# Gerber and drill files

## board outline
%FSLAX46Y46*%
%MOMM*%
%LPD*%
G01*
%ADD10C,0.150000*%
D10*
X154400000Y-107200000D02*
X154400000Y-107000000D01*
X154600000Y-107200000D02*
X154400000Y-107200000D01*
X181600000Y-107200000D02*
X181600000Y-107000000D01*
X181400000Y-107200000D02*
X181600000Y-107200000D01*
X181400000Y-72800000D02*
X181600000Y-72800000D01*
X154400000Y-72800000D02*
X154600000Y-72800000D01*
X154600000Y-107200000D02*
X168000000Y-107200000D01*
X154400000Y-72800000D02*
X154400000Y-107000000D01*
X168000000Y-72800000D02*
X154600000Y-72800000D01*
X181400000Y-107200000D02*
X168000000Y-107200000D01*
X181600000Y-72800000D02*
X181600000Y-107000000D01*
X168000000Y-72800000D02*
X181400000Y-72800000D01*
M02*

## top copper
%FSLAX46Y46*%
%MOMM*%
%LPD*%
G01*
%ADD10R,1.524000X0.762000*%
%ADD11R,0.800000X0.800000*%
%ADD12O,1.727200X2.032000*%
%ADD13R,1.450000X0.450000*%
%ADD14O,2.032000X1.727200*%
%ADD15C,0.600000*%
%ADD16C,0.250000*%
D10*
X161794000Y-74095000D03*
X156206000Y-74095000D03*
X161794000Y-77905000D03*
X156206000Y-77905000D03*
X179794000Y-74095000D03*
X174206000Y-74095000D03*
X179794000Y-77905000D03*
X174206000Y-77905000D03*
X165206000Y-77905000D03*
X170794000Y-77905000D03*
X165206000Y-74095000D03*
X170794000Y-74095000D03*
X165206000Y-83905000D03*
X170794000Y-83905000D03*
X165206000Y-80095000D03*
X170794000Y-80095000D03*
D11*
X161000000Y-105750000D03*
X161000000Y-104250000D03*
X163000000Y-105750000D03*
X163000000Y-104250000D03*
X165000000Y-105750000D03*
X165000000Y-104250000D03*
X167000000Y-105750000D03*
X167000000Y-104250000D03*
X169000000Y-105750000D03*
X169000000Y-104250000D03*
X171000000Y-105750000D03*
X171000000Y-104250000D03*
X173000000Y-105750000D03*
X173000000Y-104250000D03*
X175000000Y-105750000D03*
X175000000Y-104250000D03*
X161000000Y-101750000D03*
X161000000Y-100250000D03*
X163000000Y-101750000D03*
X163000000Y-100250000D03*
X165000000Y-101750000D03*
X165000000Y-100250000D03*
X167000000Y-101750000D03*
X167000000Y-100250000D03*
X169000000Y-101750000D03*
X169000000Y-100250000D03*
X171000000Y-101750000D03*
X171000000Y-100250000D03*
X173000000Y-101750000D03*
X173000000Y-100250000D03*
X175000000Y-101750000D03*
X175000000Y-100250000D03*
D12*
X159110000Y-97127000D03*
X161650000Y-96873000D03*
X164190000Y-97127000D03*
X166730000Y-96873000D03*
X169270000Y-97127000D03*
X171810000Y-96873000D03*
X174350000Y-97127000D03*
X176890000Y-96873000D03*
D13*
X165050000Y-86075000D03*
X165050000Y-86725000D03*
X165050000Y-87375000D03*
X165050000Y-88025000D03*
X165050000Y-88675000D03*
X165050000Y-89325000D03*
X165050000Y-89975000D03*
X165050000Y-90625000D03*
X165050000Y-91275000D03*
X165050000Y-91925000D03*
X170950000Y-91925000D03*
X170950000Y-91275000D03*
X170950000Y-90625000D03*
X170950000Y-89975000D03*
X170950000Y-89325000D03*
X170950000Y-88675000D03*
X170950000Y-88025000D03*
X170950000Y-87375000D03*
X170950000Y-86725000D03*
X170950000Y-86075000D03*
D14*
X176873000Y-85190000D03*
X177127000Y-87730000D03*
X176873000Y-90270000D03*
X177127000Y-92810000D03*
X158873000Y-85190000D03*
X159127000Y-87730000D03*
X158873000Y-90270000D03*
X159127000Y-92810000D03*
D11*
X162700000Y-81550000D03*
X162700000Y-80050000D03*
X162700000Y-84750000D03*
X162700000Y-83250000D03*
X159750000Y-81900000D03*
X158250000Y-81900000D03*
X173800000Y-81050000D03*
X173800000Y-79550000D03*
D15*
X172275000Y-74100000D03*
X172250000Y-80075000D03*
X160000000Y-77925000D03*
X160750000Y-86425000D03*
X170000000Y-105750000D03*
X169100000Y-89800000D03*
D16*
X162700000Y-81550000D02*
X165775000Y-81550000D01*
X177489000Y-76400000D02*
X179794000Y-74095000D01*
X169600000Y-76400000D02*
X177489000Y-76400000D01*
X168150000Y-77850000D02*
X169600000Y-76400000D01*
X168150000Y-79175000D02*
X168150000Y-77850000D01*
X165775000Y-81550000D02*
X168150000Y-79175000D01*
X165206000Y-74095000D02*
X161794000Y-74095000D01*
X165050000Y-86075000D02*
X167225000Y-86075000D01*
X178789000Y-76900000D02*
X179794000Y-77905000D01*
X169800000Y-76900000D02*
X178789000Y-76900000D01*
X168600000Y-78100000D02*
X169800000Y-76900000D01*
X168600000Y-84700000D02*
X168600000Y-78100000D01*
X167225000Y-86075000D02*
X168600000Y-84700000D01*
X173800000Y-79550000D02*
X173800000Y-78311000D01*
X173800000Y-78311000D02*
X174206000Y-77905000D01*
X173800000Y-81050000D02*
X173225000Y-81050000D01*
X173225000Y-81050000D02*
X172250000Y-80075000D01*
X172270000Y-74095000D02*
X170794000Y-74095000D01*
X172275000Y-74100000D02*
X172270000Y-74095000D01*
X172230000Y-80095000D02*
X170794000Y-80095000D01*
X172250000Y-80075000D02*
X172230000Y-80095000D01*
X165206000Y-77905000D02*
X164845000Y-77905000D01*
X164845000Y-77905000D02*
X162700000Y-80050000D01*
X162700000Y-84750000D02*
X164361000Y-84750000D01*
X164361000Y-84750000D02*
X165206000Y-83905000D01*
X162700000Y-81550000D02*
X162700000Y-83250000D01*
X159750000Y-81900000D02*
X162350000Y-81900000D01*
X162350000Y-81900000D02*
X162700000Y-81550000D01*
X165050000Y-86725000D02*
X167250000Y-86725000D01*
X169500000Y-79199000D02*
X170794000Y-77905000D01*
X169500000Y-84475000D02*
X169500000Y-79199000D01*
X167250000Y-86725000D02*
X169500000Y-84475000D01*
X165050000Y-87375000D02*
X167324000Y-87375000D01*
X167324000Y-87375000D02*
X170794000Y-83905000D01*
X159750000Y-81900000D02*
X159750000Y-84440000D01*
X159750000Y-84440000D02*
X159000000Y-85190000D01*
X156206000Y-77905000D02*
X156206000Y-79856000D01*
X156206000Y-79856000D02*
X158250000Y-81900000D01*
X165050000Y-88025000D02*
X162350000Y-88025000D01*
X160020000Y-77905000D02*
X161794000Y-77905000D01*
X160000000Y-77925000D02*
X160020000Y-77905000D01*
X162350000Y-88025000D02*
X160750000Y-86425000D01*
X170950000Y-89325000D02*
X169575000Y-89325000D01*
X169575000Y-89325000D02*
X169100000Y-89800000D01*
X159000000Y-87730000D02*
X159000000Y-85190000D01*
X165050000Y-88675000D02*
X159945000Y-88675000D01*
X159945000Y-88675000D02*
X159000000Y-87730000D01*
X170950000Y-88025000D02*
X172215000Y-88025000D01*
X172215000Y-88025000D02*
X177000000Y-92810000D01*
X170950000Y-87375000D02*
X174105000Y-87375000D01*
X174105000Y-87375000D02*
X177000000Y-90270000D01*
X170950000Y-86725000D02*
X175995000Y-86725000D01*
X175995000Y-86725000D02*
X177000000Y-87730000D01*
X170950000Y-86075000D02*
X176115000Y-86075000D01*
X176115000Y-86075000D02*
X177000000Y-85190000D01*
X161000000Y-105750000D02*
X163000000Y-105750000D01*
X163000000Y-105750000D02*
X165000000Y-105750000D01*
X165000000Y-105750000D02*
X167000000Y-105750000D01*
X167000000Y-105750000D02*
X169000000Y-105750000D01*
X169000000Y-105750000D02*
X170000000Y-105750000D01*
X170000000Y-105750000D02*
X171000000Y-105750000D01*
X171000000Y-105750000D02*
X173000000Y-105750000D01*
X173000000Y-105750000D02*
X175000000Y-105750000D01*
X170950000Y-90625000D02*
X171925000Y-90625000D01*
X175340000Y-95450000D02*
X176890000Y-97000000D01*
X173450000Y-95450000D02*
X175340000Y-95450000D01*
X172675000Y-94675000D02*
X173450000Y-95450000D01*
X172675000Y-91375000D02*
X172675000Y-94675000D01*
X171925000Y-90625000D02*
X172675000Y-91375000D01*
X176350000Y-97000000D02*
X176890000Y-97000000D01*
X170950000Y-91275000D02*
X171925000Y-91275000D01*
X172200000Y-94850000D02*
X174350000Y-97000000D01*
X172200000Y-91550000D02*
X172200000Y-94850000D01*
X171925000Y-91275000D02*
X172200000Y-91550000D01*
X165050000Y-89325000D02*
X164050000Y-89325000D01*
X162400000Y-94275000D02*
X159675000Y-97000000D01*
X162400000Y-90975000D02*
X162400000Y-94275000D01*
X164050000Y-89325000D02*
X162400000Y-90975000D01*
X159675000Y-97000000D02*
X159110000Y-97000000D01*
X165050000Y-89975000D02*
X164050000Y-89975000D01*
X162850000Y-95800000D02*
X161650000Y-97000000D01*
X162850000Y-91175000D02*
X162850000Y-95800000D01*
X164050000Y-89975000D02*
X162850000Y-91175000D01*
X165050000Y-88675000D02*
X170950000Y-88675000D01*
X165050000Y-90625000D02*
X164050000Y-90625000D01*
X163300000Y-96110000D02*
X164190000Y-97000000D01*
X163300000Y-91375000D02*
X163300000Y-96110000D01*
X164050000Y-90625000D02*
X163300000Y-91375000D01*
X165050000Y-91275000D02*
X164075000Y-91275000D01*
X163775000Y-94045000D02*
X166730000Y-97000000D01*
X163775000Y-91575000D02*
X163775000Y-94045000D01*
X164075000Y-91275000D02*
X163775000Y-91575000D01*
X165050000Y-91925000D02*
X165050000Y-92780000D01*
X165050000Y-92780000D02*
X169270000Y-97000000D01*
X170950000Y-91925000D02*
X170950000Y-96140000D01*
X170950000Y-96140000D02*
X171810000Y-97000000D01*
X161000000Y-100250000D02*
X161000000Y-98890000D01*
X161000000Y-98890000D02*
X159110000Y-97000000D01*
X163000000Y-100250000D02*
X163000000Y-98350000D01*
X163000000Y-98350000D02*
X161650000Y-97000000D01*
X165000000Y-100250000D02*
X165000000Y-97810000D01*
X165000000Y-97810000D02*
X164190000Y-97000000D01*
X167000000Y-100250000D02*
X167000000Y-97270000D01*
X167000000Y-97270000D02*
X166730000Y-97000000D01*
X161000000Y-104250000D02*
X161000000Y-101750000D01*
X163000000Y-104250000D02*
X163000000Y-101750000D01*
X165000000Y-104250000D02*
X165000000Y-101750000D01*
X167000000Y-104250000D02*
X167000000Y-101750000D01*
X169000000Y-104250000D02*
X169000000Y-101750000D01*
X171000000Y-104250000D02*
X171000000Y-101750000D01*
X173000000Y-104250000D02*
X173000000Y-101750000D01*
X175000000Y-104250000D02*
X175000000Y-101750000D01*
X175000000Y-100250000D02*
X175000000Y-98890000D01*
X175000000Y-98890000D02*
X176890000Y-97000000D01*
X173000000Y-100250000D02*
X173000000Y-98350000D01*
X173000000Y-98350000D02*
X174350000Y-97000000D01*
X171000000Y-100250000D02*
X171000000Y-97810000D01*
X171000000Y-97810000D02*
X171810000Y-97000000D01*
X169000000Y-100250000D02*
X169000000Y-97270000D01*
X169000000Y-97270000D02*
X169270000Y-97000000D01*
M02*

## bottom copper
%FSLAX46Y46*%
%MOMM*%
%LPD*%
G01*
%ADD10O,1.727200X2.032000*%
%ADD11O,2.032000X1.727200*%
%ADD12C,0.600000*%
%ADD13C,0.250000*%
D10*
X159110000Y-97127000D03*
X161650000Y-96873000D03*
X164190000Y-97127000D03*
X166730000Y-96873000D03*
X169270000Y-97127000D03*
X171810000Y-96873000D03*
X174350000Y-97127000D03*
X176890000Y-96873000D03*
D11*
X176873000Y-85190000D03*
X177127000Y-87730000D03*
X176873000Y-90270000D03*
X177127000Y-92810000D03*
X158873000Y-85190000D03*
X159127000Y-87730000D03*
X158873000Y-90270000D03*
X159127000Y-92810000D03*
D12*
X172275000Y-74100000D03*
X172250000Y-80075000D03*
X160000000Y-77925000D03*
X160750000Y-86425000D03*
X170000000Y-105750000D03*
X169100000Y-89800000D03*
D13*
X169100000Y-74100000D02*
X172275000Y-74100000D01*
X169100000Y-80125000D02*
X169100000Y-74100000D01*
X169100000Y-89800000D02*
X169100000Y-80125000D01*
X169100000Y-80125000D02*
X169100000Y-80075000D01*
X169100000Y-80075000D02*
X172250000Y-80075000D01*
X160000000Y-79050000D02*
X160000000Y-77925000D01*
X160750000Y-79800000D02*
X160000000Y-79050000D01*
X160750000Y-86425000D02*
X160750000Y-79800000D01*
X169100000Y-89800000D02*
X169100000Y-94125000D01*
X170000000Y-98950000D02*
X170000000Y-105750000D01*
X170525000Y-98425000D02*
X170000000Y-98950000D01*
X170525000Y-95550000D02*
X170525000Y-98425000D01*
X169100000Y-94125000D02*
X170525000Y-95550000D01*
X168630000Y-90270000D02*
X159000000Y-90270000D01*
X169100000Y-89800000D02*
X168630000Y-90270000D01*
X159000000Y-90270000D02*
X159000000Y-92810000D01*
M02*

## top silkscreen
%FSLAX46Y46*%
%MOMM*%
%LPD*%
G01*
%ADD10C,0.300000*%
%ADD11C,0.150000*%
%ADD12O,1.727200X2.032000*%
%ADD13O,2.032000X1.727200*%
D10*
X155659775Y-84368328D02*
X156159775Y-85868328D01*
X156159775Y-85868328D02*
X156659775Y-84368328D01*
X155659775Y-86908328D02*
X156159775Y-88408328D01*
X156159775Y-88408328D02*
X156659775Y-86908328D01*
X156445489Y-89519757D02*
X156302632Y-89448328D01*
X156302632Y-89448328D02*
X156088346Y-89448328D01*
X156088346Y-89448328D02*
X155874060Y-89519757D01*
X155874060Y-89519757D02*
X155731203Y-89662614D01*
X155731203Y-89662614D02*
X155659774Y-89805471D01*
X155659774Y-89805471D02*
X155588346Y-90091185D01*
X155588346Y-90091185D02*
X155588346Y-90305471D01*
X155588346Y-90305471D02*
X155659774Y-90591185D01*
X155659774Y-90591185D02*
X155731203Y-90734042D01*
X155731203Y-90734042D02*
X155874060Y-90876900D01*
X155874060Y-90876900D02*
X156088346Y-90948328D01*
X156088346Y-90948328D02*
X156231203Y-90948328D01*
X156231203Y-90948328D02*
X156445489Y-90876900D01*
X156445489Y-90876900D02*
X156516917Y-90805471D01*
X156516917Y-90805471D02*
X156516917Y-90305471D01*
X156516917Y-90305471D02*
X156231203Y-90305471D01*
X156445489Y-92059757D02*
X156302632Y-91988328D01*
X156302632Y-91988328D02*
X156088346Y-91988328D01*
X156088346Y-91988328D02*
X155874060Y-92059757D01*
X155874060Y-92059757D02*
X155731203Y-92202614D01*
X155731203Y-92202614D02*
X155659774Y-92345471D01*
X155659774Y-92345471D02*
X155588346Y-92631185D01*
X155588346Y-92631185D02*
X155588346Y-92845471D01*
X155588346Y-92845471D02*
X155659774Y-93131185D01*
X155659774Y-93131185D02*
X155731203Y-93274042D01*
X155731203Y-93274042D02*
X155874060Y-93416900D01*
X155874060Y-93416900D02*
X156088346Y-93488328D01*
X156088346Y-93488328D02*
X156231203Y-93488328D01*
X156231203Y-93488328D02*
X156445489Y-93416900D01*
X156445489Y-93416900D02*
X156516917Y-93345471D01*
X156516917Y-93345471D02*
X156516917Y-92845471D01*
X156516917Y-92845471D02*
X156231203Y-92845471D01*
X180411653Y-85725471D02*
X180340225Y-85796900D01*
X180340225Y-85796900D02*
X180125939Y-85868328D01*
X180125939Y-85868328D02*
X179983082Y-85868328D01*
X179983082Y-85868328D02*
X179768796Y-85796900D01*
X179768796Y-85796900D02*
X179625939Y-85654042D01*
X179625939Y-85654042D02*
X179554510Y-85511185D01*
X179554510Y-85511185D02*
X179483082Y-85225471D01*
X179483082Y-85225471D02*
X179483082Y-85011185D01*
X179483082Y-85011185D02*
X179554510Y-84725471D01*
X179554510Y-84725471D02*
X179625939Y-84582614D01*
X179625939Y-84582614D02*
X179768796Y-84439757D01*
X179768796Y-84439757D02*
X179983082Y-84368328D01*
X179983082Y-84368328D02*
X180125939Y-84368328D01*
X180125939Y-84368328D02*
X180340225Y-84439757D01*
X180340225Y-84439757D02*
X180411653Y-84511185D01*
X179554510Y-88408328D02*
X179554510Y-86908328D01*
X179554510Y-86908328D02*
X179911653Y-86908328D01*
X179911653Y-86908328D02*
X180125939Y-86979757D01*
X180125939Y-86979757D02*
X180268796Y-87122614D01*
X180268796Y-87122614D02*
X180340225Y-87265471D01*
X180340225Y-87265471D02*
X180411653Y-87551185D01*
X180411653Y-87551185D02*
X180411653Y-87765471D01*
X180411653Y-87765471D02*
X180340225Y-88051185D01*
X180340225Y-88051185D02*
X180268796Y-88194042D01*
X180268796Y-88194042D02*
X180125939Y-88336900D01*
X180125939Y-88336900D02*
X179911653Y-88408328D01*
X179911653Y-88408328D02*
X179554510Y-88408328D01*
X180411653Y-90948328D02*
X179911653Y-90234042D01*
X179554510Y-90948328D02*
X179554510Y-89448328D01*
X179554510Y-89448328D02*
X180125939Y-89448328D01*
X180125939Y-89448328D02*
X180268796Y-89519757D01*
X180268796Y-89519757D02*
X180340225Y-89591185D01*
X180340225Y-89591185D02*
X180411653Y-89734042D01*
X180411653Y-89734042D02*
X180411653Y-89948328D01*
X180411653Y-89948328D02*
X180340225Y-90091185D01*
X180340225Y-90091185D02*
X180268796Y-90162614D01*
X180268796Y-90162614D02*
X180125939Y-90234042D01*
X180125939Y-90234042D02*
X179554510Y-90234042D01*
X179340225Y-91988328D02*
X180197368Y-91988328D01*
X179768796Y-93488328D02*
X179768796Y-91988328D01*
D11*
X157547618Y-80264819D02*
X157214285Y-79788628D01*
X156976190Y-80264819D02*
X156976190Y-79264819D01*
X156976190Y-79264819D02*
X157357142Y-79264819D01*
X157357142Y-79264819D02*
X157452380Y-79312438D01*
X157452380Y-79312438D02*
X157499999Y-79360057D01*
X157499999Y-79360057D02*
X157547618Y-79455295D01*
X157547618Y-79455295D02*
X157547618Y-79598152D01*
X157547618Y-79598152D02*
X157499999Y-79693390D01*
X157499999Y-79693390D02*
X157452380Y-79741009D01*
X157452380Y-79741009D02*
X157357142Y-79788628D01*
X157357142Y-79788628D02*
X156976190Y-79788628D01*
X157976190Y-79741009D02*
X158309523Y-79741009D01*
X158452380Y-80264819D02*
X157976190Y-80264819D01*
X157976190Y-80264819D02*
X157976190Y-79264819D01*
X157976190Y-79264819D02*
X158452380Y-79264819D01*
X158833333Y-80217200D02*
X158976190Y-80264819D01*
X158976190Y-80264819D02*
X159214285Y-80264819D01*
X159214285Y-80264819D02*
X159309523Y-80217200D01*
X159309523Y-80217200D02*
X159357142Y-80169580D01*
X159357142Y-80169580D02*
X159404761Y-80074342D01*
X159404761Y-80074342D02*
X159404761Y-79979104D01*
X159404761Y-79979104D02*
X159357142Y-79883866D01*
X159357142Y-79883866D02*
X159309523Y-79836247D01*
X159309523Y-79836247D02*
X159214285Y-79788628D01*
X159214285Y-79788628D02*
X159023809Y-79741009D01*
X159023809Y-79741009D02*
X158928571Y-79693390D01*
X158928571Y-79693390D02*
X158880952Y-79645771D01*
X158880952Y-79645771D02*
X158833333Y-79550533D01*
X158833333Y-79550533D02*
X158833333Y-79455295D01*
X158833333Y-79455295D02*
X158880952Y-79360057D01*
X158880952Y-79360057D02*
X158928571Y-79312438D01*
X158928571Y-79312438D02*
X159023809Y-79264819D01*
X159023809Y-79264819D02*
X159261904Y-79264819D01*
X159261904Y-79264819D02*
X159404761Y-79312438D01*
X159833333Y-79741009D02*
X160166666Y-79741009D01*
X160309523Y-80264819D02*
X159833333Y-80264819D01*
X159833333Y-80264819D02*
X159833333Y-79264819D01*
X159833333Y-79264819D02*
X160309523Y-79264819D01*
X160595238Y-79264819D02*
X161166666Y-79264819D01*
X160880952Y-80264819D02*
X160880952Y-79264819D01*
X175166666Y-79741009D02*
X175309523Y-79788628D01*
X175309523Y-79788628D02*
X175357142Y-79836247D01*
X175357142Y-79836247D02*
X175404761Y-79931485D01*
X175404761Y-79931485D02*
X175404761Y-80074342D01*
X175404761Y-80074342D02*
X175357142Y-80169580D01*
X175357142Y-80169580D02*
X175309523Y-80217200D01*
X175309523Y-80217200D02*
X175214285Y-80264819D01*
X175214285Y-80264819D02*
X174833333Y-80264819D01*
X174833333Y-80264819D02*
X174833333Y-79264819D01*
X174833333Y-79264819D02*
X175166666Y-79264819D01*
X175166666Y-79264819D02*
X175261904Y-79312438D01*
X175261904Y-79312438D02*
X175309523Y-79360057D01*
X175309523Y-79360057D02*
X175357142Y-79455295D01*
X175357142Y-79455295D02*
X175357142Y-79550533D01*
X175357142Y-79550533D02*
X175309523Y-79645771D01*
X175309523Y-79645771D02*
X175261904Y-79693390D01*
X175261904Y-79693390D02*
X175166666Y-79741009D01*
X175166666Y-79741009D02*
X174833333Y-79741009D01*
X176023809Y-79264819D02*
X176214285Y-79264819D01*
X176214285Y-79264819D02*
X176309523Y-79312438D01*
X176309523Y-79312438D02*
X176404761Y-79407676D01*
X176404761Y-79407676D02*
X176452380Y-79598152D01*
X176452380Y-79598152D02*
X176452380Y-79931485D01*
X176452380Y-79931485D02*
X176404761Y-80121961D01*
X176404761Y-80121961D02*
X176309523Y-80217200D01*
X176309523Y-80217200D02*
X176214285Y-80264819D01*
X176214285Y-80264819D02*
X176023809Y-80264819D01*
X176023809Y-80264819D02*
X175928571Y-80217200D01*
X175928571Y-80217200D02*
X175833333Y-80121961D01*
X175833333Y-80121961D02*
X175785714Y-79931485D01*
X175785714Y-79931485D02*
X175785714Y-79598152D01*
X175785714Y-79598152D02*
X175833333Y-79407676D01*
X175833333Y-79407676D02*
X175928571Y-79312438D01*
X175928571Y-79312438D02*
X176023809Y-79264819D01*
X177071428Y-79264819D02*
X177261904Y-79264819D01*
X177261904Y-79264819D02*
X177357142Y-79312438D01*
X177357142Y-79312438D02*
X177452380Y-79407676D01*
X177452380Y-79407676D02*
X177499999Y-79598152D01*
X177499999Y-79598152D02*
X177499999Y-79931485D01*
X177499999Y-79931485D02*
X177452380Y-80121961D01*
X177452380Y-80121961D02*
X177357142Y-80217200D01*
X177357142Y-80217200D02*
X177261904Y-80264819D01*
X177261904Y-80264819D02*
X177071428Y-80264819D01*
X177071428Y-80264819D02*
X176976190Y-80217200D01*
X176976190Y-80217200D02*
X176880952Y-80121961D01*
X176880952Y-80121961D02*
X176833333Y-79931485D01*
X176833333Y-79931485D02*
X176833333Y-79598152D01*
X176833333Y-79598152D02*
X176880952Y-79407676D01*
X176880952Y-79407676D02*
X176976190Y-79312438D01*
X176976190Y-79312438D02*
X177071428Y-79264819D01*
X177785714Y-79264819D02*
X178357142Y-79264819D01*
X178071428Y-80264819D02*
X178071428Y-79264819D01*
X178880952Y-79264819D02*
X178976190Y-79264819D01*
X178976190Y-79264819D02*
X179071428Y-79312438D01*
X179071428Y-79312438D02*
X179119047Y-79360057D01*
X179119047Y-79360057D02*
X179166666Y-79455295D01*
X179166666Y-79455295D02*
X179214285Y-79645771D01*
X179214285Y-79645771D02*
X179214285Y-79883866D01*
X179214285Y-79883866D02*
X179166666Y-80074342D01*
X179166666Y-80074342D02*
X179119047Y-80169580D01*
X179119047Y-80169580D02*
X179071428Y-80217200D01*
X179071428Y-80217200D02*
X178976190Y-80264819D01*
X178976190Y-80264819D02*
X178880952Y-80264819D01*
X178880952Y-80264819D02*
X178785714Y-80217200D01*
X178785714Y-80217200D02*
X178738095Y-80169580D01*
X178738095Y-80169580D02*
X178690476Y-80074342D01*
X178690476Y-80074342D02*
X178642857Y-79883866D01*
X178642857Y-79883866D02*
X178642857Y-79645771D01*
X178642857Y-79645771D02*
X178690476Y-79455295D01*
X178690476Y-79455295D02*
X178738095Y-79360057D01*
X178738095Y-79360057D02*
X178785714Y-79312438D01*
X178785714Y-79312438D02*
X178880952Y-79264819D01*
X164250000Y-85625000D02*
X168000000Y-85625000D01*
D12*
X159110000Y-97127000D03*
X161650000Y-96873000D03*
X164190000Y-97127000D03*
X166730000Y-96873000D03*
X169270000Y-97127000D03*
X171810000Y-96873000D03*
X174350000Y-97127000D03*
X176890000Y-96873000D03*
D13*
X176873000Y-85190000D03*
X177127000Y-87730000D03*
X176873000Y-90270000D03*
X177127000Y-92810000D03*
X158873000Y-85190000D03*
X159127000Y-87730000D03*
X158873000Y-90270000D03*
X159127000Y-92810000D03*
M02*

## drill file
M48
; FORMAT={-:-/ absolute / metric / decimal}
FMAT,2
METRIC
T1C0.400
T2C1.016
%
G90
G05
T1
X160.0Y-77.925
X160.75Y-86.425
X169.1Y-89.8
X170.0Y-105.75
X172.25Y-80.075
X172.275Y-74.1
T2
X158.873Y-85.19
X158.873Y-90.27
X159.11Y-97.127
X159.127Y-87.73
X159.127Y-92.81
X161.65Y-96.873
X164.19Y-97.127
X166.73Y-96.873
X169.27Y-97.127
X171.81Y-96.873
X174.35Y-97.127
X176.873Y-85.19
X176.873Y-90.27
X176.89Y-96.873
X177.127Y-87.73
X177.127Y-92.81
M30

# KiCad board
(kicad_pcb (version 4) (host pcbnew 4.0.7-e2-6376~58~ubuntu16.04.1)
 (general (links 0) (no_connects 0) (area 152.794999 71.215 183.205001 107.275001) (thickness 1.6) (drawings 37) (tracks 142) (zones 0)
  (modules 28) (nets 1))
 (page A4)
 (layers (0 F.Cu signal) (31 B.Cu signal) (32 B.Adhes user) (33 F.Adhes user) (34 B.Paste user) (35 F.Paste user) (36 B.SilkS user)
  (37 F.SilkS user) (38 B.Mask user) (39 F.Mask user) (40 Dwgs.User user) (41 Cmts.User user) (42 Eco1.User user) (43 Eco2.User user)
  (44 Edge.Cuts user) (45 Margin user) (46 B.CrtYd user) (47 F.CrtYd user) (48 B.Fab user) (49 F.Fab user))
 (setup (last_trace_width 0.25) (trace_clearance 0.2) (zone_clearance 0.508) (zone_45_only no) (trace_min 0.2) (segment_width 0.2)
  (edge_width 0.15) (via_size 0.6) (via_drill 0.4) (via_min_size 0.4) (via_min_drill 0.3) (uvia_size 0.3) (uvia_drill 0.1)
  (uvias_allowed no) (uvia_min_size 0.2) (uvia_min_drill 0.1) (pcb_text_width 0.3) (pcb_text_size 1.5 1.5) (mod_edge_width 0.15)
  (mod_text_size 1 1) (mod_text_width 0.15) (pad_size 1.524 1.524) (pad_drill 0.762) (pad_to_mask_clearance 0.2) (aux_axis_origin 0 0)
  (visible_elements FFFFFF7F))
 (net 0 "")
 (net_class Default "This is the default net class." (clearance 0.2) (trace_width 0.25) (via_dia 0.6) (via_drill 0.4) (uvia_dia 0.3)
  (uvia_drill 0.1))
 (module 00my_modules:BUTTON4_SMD (layer F.Cu) (at 159 76 180)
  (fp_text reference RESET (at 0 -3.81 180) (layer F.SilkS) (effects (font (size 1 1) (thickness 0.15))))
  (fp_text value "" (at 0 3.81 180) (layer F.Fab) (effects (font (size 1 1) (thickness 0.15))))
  (pad 1 smd rect (at -2.794 1.905 180) (size 1.524 0.762) (layers F.Cu F.Paste F.Mask))
  (pad 2 smd rect (at 2.794 1.905 180) (size 1.524 0.762) (layers F.Cu F.Paste F.Mask))
  (pad 3 smd rect (at -2.794 -1.905 180) (size 1.524 0.762) (layers F.Cu F.Paste F.Mask))
  (pad 4 smd rect (at 2.794 -1.905 180) (size 1.524 0.762) (layers F.Cu F.Paste F.Mask)))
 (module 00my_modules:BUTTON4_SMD (layer F.Cu) (at 177 76 180)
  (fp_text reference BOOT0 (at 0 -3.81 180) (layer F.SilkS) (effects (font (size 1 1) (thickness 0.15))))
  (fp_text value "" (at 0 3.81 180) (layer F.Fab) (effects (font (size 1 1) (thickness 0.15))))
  (pad 1 smd rect (at -2.794 1.905 180) (size 1.524 0.762) (layers F.Cu F.Paste F.Mask))
  (pad 2 smd rect (at 2.794 1.905 180) (size 1.524 0.762) (layers F.Cu F.Paste F.Mask))
  (pad 3 smd rect (at -2.794 -1.905 180) (size 1.524 0.762) (layers F.Cu F.Paste F.Mask))
  (pad 4 smd rect (at 2.794 -1.905 180) (size 1.524 0.762) (layers F.Cu F.Paste F.Mask)))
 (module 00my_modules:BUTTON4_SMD (layer F.Cu) (at 168 76)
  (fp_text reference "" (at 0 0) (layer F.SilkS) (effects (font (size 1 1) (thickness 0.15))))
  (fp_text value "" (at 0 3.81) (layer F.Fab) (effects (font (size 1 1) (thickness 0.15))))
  (pad 1 smd rect (at -2.794 1.905) (size 1.524 0.762) (layers F.Cu F.Paste F.Mask))
  (pad 2 smd rect (at 2.794 1.905) (size 1.524 0.762) (layers F.Cu F.Paste F.Mask))
  (pad 3 smd rect (at -2.794 -1.905) (size 1.524 0.762) (layers F.Cu F.Paste F.Mask))
  (pad 4 smd rect (at 2.794 -1.905) (size 1.524 0.762) (layers F.Cu F.Paste F.Mask)))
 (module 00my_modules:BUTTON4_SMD (layer F.Cu) (at 168 82)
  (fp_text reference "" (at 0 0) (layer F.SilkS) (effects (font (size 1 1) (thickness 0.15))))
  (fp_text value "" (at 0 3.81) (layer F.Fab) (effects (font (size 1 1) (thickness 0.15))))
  (pad 1 smd rect (at -2.794 1.905) (size 1.524 0.762) (layers F.Cu F.Paste F.Mask))
  (pad 2 smd rect (at 2.794 1.905) (size 1.524 0.762) (layers F.Cu F.Paste F.Mask))
  (pad 3 smd rect (at -2.794 -1.905) (size 1.524 0.762) (layers F.Cu F.Paste F.Mask))
  (pad 4 smd rect (at 2.794 -1.905) (size 1.524 0.762) (layers F.Cu F.Paste F.Mask)))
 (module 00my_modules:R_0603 (layer F.Cu) (at 161 105 90)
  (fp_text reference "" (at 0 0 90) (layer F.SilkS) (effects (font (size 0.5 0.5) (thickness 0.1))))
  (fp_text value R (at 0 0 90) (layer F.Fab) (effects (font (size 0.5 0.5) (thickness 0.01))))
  (pad 1 smd rect (at -0.75 0 90) (size 0.8 0.8) (layers F.Cu F.Paste F.Mask))
  (pad 2 smd rect (at 0.75 0 90) (size 0.8 0.8) (layers F.Cu F.Paste F.Mask)))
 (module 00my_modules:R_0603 (layer F.Cu) (at 163 105 90)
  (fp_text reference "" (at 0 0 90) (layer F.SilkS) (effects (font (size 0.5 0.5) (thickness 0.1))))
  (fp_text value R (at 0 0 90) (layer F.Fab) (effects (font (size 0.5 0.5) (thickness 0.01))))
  (pad 1 smd rect (at -0.75 0 90) (size 0.8 0.8) (layers F.Cu F.Paste F.Mask))
  (pad 2 smd rect (at 0.75 0 90) (size 0.8 0.8) (layers F.Cu F.Paste F.Mask)))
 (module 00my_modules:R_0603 (layer F.Cu) (at 165 105 90)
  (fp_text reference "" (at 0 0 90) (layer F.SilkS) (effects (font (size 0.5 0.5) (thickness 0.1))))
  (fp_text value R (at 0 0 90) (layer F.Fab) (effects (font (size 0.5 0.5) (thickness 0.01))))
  (pad 1 smd rect (at -0.75 0 90) (size 0.8 0.8) (layers F.Cu F.Paste F.Mask))
  (pad 2 smd rect (at 0.75 0 90) (size 0.8 0.8) (layers F.Cu F.Paste F.Mask)))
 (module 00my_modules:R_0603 (layer F.Cu) (at 167 105 90)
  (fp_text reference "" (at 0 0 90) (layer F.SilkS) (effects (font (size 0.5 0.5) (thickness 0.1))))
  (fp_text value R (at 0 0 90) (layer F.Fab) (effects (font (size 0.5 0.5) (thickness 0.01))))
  (pad 1 smd rect (at -0.75 0 90) (size 0.8 0.8) (layers F.Cu F.Paste F.Mask))
  (pad 2 smd rect (at 0.75 0 90) (size 0.8 0.8) (layers F.Cu F.Paste F.Mask)))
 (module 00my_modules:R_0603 (layer F.Cu) (at 169 105 90)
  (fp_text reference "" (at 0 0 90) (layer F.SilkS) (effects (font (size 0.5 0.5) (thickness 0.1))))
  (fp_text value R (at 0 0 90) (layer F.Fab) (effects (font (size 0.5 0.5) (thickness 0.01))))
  (pad 1 smd rect (at -0.75 0 90) (size 0.8 0.8) (layers F.Cu F.Paste F.Mask))
  (pad 2 smd rect (at 0.75 0 90) (size 0.8 0.8) (layers F.Cu F.Paste F.Mask)))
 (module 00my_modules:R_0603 (layer F.Cu) (at 171 105 90)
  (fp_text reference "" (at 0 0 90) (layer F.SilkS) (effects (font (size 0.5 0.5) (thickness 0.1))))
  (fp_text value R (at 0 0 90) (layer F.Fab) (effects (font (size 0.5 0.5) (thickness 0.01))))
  (pad 1 smd rect (at -0.75 0 90) (size 0.8 0.8) (layers F.Cu F.Paste F.Mask))
  (pad 2 smd rect (at 0.75 0 90) (size 0.8 0.8) (layers F.Cu F.Paste F.Mask)))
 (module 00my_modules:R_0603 (layer F.Cu) (at 173 105 90)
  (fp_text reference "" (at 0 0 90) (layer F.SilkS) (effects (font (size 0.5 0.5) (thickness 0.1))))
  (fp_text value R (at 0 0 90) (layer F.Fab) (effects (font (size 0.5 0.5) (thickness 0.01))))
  (pad 1 smd rect (at -0.75 0 90) (size 0.8 0.8) (layers F.Cu F.Paste F.Mask))
  (pad 2 smd rect (at 0.75 0 90) (size 0.8 0.8) (layers F.Cu F.Paste F.Mask)))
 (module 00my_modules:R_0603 (layer F.Cu) (at 175 105 90)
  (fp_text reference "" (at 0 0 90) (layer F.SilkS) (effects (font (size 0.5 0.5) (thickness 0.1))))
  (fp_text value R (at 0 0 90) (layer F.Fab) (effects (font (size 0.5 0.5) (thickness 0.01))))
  (pad 1 smd rect (at -0.75 0 90) (size 0.8 0.8) (layers F.Cu F.Paste F.Mask))
  (pad 2 smd rect (at 0.75 0 90) (size 0.8 0.8) (layers F.Cu F.Paste F.Mask)))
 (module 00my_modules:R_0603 (layer F.Cu) (at 161 101 90)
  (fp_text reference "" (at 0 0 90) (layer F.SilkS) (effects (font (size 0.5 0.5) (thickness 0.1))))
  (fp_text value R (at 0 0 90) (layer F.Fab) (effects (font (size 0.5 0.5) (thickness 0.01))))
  (pad 1 smd rect (at -0.75 0 90) (size 0.8 0.8) (layers F.Cu F.Paste F.Mask))
  (pad 2 smd rect (at 0.75 0 90) (size 0.8 0.8) (layers F.Cu F.Paste F.Mask)))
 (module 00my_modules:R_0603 (layer F.Cu) (at 163 101 90)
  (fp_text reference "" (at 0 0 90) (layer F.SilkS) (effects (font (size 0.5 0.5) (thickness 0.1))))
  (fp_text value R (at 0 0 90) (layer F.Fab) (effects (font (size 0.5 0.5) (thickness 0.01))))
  (pad 1 smd rect (at -0.75 0 90) (size 0.8 0.8) (layers F.Cu F.Paste F.Mask))
  (pad 2 smd rect (at 0.75 0 90) (size 0.8 0.8) (layers F.Cu F.Paste F.Mask)))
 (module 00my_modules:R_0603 (layer F.Cu) (at 165 101 90)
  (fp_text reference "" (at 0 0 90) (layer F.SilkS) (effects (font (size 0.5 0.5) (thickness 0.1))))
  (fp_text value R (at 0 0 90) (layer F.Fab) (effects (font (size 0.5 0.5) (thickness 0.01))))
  (pad 1 smd rect (at -0.75 0 90) (size 0.8 0.8) (layers F.Cu F.Paste F.Mask))
  (pad 2 smd rect (at 0.75 0 90) (size 0.8 0.8) (layers F.Cu F.Paste F.Mask)))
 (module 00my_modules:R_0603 (layer F.Cu) (at 167 101 90)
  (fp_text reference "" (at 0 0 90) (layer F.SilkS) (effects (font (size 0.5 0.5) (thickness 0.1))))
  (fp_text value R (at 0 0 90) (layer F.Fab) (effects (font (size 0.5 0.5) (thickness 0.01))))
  (pad 1 smd rect (at -0.75 0 90) (size 0.8 0.8) (layers F.Cu F.Paste F.Mask))
  (pad 2 smd rect (at 0.75 0 90) (size 0.8 0.8) (layers F.Cu F.Paste F.Mask)))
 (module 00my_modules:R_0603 (layer F.Cu) (at 169 101 90)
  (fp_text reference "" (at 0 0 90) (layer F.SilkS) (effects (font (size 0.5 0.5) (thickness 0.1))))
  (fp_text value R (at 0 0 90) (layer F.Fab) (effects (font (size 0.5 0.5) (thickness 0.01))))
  (pad 1 smd rect (at -0.75 0 90) (size 0.8 0.8) (layers F.Cu F.Paste F.Mask))
  (pad 2 smd rect (at 0.75 0 90) (size 0.8 0.8) (layers F.Cu F.Paste F.Mask)))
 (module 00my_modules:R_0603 (layer F.Cu) (at 171 101 90)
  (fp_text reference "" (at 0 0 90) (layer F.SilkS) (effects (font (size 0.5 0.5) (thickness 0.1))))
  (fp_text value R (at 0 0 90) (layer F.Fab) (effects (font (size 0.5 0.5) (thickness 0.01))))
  (pad 1 smd rect (at -0.75 0 90) (size 0.8 0.8) (layers F.Cu F.Paste F.Mask))
  (pad 2 smd rect (at 0.75 0 90) (size 0.8 0.8) (layers F.Cu F.Paste F.Mask)))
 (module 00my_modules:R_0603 (layer F.Cu) (at 173 101 90)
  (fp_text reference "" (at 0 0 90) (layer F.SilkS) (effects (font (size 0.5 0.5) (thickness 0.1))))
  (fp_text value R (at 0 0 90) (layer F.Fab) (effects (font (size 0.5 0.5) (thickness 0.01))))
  (pad 1 smd rect (at -0.75 0 90) (size 0.8 0.8) (layers F.Cu F.Paste F.Mask))
  (pad 2 smd rect (at 0.75 0 90) (size 0.8 0.8) (layers F.Cu F.Paste F.Mask)))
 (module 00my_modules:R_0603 (layer F.Cu) (at 175 101 90)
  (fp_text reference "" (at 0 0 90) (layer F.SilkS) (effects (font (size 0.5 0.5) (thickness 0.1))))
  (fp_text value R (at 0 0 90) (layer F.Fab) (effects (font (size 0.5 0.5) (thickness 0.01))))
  (pad 1 smd rect (at -0.75 0 90) (size 0.8 0.8) (layers F.Cu F.Paste F.Mask))
  (pad 2 smd rect (at 0.75 0 90) (size 0.8 0.8) (layers F.Cu F.Paste F.Mask)))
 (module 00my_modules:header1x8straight (layer F.Cu) (at 168 97 90)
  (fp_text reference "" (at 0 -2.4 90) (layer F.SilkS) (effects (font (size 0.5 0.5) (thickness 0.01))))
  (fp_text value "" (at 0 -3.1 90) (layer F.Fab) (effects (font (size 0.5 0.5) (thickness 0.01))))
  (pad 1 thru_hole oval (at -0.127 -8.89 90) (size 2.032 1.7272) (drill 1.016) (layers *.Cu *.Mask F.SilkS))
  (pad 2 thru_hole oval (at 0.127 -6.35 90) (size 2.032 1.7272) (drill 1.016) (layers *.Cu *.Mask F.SilkS))
  (pad 3 thru_hole oval (at -0.127 -3.81 90) (size 2.032 1.7272) (drill 1.016) (layers *.Cu *.Mask F.SilkS))
  (pad 4 thru_hole oval (at 0.127 -1.27 90) (size 2.032 1.7272) (drill 1.016) (layers *.Cu *.Mask F.SilkS))
  (pad 5 thru_hole oval (at -0.127 1.27 90) (size 2.032 1.7272) (drill 1.016) (layers *.Cu *.Mask F.SilkS))
  (pad 6 thru_hole oval (at 0.127 3.81 90) (size 2.032 1.7272) (drill 1.016) (layers *.Cu *.Mask F.SilkS))
  (pad 7 thru_hole oval (at -0.127 6.35 90) (size 2.032 1.7272) (drill 1.016) (layers *.Cu *.Mask F.SilkS))
  (pad 8 thru_hole oval (at 0.127 8.89 90) (size 2.032 1.7272) (drill 1.016) (layers *.Cu *.Mask F.SilkS)))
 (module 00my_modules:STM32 (layer F.Cu) (at 168 89)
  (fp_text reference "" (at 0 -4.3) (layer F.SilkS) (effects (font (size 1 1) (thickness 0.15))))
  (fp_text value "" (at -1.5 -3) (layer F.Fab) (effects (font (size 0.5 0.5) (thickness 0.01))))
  (fp_line (start -3.75 -3.375) (end 0 -3.375) (layer F.SilkS) (width 0.15))
  (pad BOOT smd rect (at -2.95 -2.925) (size 1.45 0.45) (layers F.Cu F.Paste F.Mask))
  (pad 2 smd rect (at -2.95 -2.275) (size 1.45 0.45) (layers F.Cu F.Paste F.Mask))
  (pad 3 smd rect (at -2.95 -1.625) (size 1.45 0.45) (layers F.Cu F.Paste F.Mask))
  (pad NRST smd rect (at -2.95 -0.975) (size 1.45 0.45) (layers F.Cu F.Paste F.Mask))
  (pad VCC smd rect (at -2.95 -0.325) (size 1.45 0.45) (layers F.Cu F.Paste F.Mask))
  (pad PA0 smd rect (at -2.95 0.325) (size 1.45 0.45) (layers F.Cu F.Paste F.Mask))
  (pad PA1 smd rect (at -2.95 0.975) (size 1.45 0.45) (layers F.Cu F.Paste F.Mask))
  (pad PA2 smd rect (at -2.95 1.625) (size 1.45 0.45) (layers F.Cu F.Paste F.Mask))
  (pad PA3 smd rect (at -2.95 2.275) (size 1.45 0.45) (layers F.Cu F.Paste F.Mask))
  (pad PA4 smd rect (at -2.95 2.925) (size 1.45 0.45) (layers F.Cu F.Paste F.Mask))
  (pad PA5 smd rect (at 2.95 2.925) (size 1.45 0.45) (layers F.Cu F.Paste F.Mask))
  (pad PA6 smd rect (at 2.95 2.275) (size 1.45 0.45) (layers F.Cu F.Paste F.Mask))
  (pad PA7 smd rect (at 2.95 1.625) (size 1.45 0.45) (layers F.Cu F.Paste F.Mask))
  (pad PB1 smd rect (at 2.95 0.975) (size 1.45 0.45) (layers F.Cu F.Paste F.Mask))
  (pad GND smd rect (at 2.95 0.325) (size 1.45 0.45) (layers F.Cu F.Paste F.Mask))
  (pad VCC smd rect (at 2.95 -0.325) (size 1.45 0.45) (layers F.Cu F.Paste F.Mask))
  (pad TX smd rect (at 2.95 -0.975) (size 1.45 0.45) (layers F.Cu F.Paste F.Mask))
  (pad RX smd rect (at 2.95 -1.625) (size 1.45 0.45) (layers F.Cu F.Paste F.Mask))
  (pad DIO smd rect (at 2.95 -2.275) (size 1.45 0.45) (layers F.Cu F.Paste F.Mask))
  (pad CLK smd rect (at 2.95 -2.925) (size 1.45 0.45) (layers F.Cu F.Paste F.Mask)))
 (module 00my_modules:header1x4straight (layer F.Cu) (at 177 89)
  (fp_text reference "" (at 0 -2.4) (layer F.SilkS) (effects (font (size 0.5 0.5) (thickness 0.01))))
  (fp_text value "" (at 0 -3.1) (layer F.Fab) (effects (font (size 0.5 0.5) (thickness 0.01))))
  (pad 1 thru_hole oval (at -0.127 -3.81) (size 2.032 1.7272) (drill 1.016) (layers *.Cu *.Mask F.SilkS))
  (pad 2 thru_hole oval (at 0.127 -1.27) (size 2.032 1.7272) (drill 1.016) (layers *.Cu *.Mask F.SilkS))
  (pad 3 thru_hole oval (at -0.127 1.27) (size 2.032 1.7272) (drill 1.016) (layers *.Cu *.Mask F.SilkS))
  (pad 4 thru_hole oval (at 0.127 3.81) (size 2.032 1.7272) (drill 1.016) (layers *.Cu *.Mask F.SilkS)))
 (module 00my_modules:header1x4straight (layer F.Cu) (at 159 89)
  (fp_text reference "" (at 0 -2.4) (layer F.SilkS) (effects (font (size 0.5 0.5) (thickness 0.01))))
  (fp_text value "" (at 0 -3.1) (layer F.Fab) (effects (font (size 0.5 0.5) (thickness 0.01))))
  (pad 1 thru_hole oval (at -0.127 -3.81) (size 2.032 1.7272) (drill 1.016) (layers *.Cu *.Mask F.SilkS))
  (pad 2 thru_hole oval (at 0.127 -1.27) (size 2.032 1.7272) (drill 1.016) (layers *.Cu *.Mask F.SilkS))
  (pad 3 thru_hole oval (at -0.127 1.27) (size 2.032 1.7272) (drill 1.016) (layers *.Cu *.Mask F.SilkS))
  (pad 4 thru_hole oval (at 0.127 3.81) (size 2.032 1.7272) (drill 1.016) (layers *.Cu *.Mask F.SilkS)))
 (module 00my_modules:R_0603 (layer F.Cu) (at 162.7 80.8 90)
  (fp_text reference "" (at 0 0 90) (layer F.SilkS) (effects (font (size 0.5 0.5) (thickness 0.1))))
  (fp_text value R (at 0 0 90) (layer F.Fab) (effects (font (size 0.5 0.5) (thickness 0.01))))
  (pad 1 smd rect (at -0.75 0 90) (size 0.8 0.8) (layers F.Cu F.Paste F.Mask))
  (pad 2 smd rect (at 0.75 0 90) (size 0.8 0.8) (layers F.Cu F.Paste F.Mask)))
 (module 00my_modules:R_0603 (layer F.Cu) (at 162.7 84 90)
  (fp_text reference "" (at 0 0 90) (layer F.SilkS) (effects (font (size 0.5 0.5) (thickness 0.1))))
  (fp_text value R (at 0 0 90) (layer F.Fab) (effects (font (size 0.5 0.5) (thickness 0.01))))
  (pad 1 smd rect (at -0.75 0 90) (size 0.8 0.8) (layers F.Cu F.Paste F.Mask))
  (pad 2 smd rect (at 0.75 0 90) (size 0.8 0.8) (layers F.Cu F.Paste F.Mask)))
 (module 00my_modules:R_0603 (layer F.Cu) (at 159 81.9 180)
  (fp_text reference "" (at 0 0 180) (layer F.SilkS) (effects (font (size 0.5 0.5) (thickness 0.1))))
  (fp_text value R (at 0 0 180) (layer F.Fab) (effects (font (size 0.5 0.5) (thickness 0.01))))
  (pad 1 smd rect (at -0.75 0 180) (size 0.8 0.8) (layers F.Cu F.Paste F.Mask))
  (pad 2 smd rect (at 0.75 0 180) (size 0.8 0.8) (layers F.Cu F.Paste F.Mask)))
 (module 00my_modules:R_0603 (layer F.Cu) (at 173.8 80.3 90)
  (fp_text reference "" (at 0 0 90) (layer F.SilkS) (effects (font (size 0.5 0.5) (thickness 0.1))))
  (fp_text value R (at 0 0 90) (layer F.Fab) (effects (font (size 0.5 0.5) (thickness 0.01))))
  (pad 1 smd rect (at -0.75 0 90) (size 0.8 0.8) (layers F.Cu F.Paste F.Mask))
  (pad 2 smd rect (at 0.75 0 90) (size 0.8 0.8) (layers F.Cu F.Paste F.Mask)))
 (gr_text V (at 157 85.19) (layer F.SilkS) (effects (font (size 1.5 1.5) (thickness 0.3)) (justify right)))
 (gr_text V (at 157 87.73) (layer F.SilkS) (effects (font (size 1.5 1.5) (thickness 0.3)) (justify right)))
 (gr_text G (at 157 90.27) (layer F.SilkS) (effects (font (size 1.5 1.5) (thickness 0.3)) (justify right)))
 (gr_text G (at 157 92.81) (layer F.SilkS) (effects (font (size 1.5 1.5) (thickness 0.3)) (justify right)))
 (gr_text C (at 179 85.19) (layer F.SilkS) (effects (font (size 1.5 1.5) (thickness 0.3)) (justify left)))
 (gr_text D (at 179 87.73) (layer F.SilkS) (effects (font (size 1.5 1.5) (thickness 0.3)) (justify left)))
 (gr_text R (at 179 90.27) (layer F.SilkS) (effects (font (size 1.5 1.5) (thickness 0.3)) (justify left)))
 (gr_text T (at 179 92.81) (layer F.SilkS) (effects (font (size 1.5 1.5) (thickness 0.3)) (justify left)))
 (gr_line (start 154.4 107.2) (end 154.4 107) (angle 90) (layer Edge.Cuts) (width 0.15))
 (gr_line (start 154.6 107.2) (end 154.4 107.2) (angle 90) (layer Edge.Cuts) (width 0.15))
 (gr_line (start 181.6 107.2) (end 181.6 107) (angle 90) (layer Edge.Cuts) (width 0.15))
 (gr_line (start 181.4 107.2) (end 181.6 107.2) (angle 90) (layer Edge.Cuts) (width 0.15))
 (gr_line (start 181.4 72.8) (end 181.6 72.8) (angle 90) (layer Edge.Cuts) (width 0.15))
 (gr_line (start 154.4 72.8) (end 154.6 72.8) (angle 90) (layer Edge.Cuts) (width 0.15))
 (gr_line (start 154.6 107.2) (end 168 107.2) (angle 90) (layer Edge.Cuts) (width 0.15))
 (gr_line (start 154.4 72.8) (end 154.4 107) (angle 90) (layer Edge.Cuts) (width 0.15))
 (gr_line (start 168 72.8) (end 154.6 72.8) (angle 90) (layer Edge.Cuts) (width 0.15))
 (gr_line (start 181.4 107.2) (end 168 107.2) (angle 90) (layer Edge.Cuts) (width 0.15))
 (gr_line (start 181.6 72.8) (end 181.6 107) (angle 90) (layer Edge.Cuts) (width 0.15))
 (gr_line (start 168 72.8) (end 181.4 72.8) (angle 90) (layer Edge.Cuts) (width 0.15))
 (segment (start 162.7 81.55) (end 165.775 81.55) (width 0.25) (layer F.Cu) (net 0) (status 400000))
 (segment (start 177.489 76.4) (end 179.794 74.095) (width 0.25) (layer F.Cu) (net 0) (status 800000))
 (segment (start 169.6 76.4) (end 177.489 76.4) (width 0.25) (layer F.Cu) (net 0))
 (segment (start 168.15 77.85) (end 169.6 76.4) (width 0.25) (layer F.Cu) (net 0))
 (segment (start 168.15 79.175) (end 168.15 77.85) (width 0.25) (layer F.Cu) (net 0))
 (segment (start 165.775 81.55) (end 168.15 79.175) (width 0.25) (layer F.Cu) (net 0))
 (segment (start 165.206 74.095) (end 161.794 74.095) (width 0.25) (layer F.Cu) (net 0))
 (segment (start 165.05 86.075) (end 167.225 86.075) (width 0.25) (layer F.Cu) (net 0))
 (segment (start 178.789 76.9) (end 179.794 77.905) (width 0.25) (layer F.Cu) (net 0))
 (segment (start 169.8 76.9) (end 178.789 76.9) (width 0.25) (layer F.Cu) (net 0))
 (segment (start 168.6 78.1) (end 169.8 76.9) (width 0.25) (layer F.Cu) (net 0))
 (segment (start 168.6 84.7) (end 168.6 78.1) (width 0.25) (layer F.Cu) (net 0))
 (segment (start 167.225 86.075) (end 168.6 84.7) (width 0.25) (layer F.Cu) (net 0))
 (segment (start 173.8 79.55) (end 173.8 78.311) (width 0.25) (layer F.Cu) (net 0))
 (segment (start 173.8 78.311) (end 174.206 77.905) (width 0.25) (layer F.Cu) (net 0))
 (segment (start 173.8 81.05) (end 173.225 81.05) (width 0.25) (layer F.Cu) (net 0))
 (segment (start 173.225 81.05) (end 172.25 80.075) (width 0.25) (layer F.Cu) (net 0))
 (segment (start 169.1 74.1) (end 172.275 74.1) (width 0.25) (layer B.Cu) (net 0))
 (segment (start 169.1 80.125) (end 169.1 74.1) (width 0.25) (layer B.Cu) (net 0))
 (segment (start 172.27 74.095) (end 170.794 74.095) (width 0.25) (layer F.Cu) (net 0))
 (segment (start 172.275 74.1) (end 172.27 74.095) (width 0.25) (layer F.Cu) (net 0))
 (via (at 172.275 74.1) (size 0.6) (drill 0.4) (layers F.Cu B.Cu) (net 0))
 (segment (start 169.1 89.8) (end 169.1 80.125) (width 0.25) (layer B.Cu) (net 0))
 (segment (start 169.1 80.125) (end 169.1 80.075) (width 0.25) (layer B.Cu) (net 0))
 (segment (start 172.23 80.095) (end 170.794 80.095) (width 0.25) (layer F.Cu) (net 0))
 (segment (start 172.25 80.075) (end 172.23 80.095) (width 0.25) (layer F.Cu) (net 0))
 (via (at 172.25 80.075) (size 0.6) (drill 0.4) (layers F.Cu B.Cu) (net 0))
 (segment (start 169.1 80.075) (end 172.25 80.075) (width 0.25) (layer B.Cu) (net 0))
 (segment (start 165.206 77.905) (end 164.845 77.905) (width 0.25) (layer F.Cu) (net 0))
 (segment (start 164.845 77.905) (end 162.7 80.05) (width 0.25) (layer F.Cu) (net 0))
 (segment (start 162.7 84.75) (end 164.361 84.75) (width 0.25) (layer F.Cu) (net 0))
 (segment (start 164.361 84.75) (end 165.206 83.905) (width 0.25) (layer F.Cu) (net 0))
 (segment (start 162.7 81.55) (end 162.7 83.25) (width 0.25) (layer F.Cu) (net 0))
 (segment (start 159.75 81.9) (end 162.35 81.9) (width 0.25) (layer F.Cu) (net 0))
 (segment (start 162.35 81.9) (end 162.7 81.55) (width 0.25) (layer F.Cu) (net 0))
 (segment (start 165.05 86.725) (end 167.25 86.725) (width 0.25) (layer F.Cu) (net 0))
 (segment (start 169.5 79.199) (end 170.794 77.905) (width 0.25) (layer F.Cu) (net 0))
 (segment (start 169.5 84.475) (end 169.5 79.199) (width 0.25) (layer F.Cu) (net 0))
 (segment (start 167.25 86.725) (end 169.5 84.475) (width 0.25) (layer F.Cu) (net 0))
 (segment (start 165.05 87.375) (end 167.324 87.375) (width 0.25) (layer F.Cu) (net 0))
 (segment (start 167.324 87.375) (end 170.794 83.905) (width 0.25) (layer F.Cu) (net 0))
 (segment (start 159.75 81.9) (end 159.75 84.44) (width 0.25) (layer F.Cu) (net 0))
 (segment (start 159.75 84.44) (end 159 85.19) (width 0.25) (layer F.Cu) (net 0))
 (segment (start 156.206 77.905) (end 156.206 79.856) (width 0.25) (layer F.Cu) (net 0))
 (segment (start 156.206 79.856) (end 158.25 81.9) (width 0.25) (layer F.Cu) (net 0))
 (segment (start 165.05 88.025) (end 162.35 88.025) (width 0.25) (layer F.Cu) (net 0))
 (segment (start 160.02 77.905) (end 161.794 77.905) (width 0.25) (layer F.Cu) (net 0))
 (segment (start 160 77.925) (end 160.02 77.905) (width 0.25) (layer F.Cu) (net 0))
 (via (at 160 77.925) (size 0.6) (drill 0.4) (layers F.Cu B.Cu) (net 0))
 (segment (start 160 79.05) (end 160 77.925) (width 0.25) (layer B.Cu) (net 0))
 (segment (start 160.75 79.8) (end 160 79.05) (width 0.25) (layer B.Cu) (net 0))
 (segment (start 160.75 86.425) (end 160.75 79.8) (width 0.25) (layer B.Cu) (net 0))
 (via (at 160.75 86.425) (size 0.6) (drill 0.4) (layers F.Cu B.Cu) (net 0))
 (segment (start 162.35 88.025) (end 160.75 86.425) (width 0.25) (layer F.Cu) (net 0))
 (segment (start 169.1 89.8) (end 169.1 94.125) (width 0.25) (layer B.Cu) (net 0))
 (via (at 170 105.75) (size 0.6) (drill 0.4) (layers F.Cu B.Cu) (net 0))
 (segment (start 170 98.95) (end 170 105.75) (width 0.25) (layer B.Cu) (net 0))
 (segment (start 170.525 98.425) (end 170 98.95) (width 0.25) (layer B.Cu) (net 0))
 (segment (start 170.525 95.55) (end 170.525 98.425) (width 0.25) (layer B.Cu) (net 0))
 (segment (start 169.1 94.125) (end 170.525 95.55) (width 0.25) (layer B.Cu) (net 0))
 (segment (start 170.95 89.325) (end 169.575 89.325) (width 0.25) (layer F.Cu) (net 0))
 (segment (start 168.63 90.27) (end 159 90.27) (width 0.25) (layer B.Cu) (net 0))
 (segment (start 169.1 89.8) (end 168.63 90.27) (width 0.25) (layer B.Cu) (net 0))
 (via (at 169.1 89.8) (size 0.6) (drill 0.4) (layers F.Cu B.Cu) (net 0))
 (segment (start 169.575 89.325) (end 169.1 89.8) (width 0.25) (layer F.Cu) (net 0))
 (segment (start 159 90.27) (end 159 92.81) (width 0.25) (layer B.Cu) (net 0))
 (segment (start 159 87.73) (end 159 85.19) (width 0.25) (layer F.Cu) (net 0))
 (segment (start 165.05 88.675) (end 159.945 88.675) (width 0.25) (layer F.Cu) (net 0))
 (segment (start 159.945 88.675) (end 159 87.73) (width 0.25) (layer F.Cu) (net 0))
 (segment (start 170.95 88.025) (end 172.215 88.025) (width 0.25) (layer F.Cu) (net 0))
 (segment (start 172.215 88.025) (end 177 92.81) (width 0.25) (layer F.Cu) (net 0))
 (segment (start 170.95 87.375) (end 174.105 87.375) (width 0.25) (layer F.Cu) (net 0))
 (segment (start 174.105 87.375) (end 177 90.27) (width 0.25) (layer F.Cu) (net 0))
 (segment (start 170.95 86.725) (end 175.995 86.725) (width 0.25) (layer F.Cu) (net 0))
 (segment (start 175.995 86.725) (end 177 87.73) (width 0.25) (layer F.Cu) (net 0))
 (segment (start 170.95 86.075) (end 176.115 86.075) (width 0.25) (layer F.Cu) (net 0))
 (segment (start 176.115 86.075) (end 177 85.19) (width 0.25) (layer F.Cu) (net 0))
 (segment (start 161 105.75) (end 163 105.75) (width 0.25) (layer F.Cu) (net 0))
 (segment (start 163 105.75) (end 165 105.75) (width 0.25) (layer F.Cu) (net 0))
 (segment (start 165 105.75) (end 167 105.75) (width 0.25) (layer F.Cu) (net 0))
 (segment (start 167 105.75) (end 169 105.75) (width 0.25) (layer F.Cu) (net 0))
 (segment (start 169 105.75) (end 170 105.75) (width 0.25) (layer F.Cu) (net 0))
 (segment (start 170 105.75) (end 171 105.75) (width 0.25) (layer F.Cu) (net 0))
 (segment (start 171 105.75) (end 173 105.75) (width 0.25) (layer F.Cu) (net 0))
 (segment (start 173 105.75) (end 175 105.75) (width 0.25) (layer F.Cu) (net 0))
 (segment (start 170.95 90.625) (end 171.925 90.625) (width 0.25) (layer F.Cu) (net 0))
 (segment (start 175.34 95.45) (end 176.89 97) (width 0.25) (layer F.Cu) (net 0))
 (segment (start 173.45 95.45) (end 175.34 95.45) (width 0.25) (layer F.Cu) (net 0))
 (segment (start 172.675 94.675) (end 173.45 95.45) (width 0.25) (layer F.Cu) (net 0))
 (segment (start 172.675 91.375) (end 172.675 94.675) (width 0.25) (layer F.Cu) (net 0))
 (segment (start 171.925 90.625) (end 172.675 91.375) (width 0.25) (layer F.Cu) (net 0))
 (segment (start 176.35 97) (end 176.89 97) (width 0.25) (layer F.Cu) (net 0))
 (segment (start 170.95 91.275) (end 171.925 91.275) (width 0.25) (layer F.Cu) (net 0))
 (segment (start 172.2 94.85) (end 174.35 97) (width 0.25) (layer F.Cu) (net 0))
 (segment (start 172.2 91.55) (end 172.2 94.85) (width 0.25) (layer F.Cu) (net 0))
 (segment (start 171.925 91.275) (end 172.2 91.55) (width 0.25) (layer F.Cu) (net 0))
 (segment (start 165.05 89.325) (end 164.05 89.325) (width 0.25) (layer F.Cu) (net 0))
 (segment (start 162.4 94.275) (end 159.675 97) (width 0.25) (layer F.Cu) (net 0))
 (segment (start 162.4 90.975) (end 162.4 94.275) (width 0.25) (layer F.Cu) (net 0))
 (segment (start 164.05 89.325) (end 162.4 90.975) (width 0.25) (layer F.Cu) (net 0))
 (segment (start 159.675 97) (end 159.11 97) (width 0.25) (layer F.Cu) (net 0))
 (segment (start 165.05 89.975) (end 164.05 89.975) (width 0.25) (layer F.Cu) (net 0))
 (segment (start 162.85 95.8) (end 161.65 97) (width 0.25) (layer F.Cu) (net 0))
 (segment (start 162.85 91.175) (end 162.85 95.8) (width 0.25) (layer F.Cu) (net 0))
 (segment (start 164.05 89.975) (end 162.85 91.175) (width 0.25) (layer F.Cu) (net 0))
 (segment (start 165.05 88.675) (end 170.95 88.675) (width 0.25) (layer F.Cu) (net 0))
 (segment (start 165.05 90.625) (end 164.05 90.625) (width 0.25) (layer F.Cu) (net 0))
 (segment (start 163.3 96.11) (end 164.19 97) (width 0.25) (layer F.Cu) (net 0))
 (segment (start 163.3 91.375) (end 163.3 96.11) (width 0.25) (layer F.Cu) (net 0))
 (segment (start 164.05 90.625) (end 163.3 91.375) (width 0.25) (layer F.Cu) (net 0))
 (segment (start 165.05 91.275) (end 164.075 91.275) (width 0.25) (layer F.Cu) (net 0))
 (segment (start 163.775 94.045) (end 166.73 97) (width 0.25) (layer F.Cu) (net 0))
 (segment (start 163.775 91.575) (end 163.775 94.045) (width 0.25) (layer F.Cu) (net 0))
 (segment (start 164.075 91.275) (end 163.775 91.575) (width 0.25) (layer F.Cu) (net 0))
 (segment (start 165.05 91.925) (end 165.05 92.78) (width 0.25) (layer F.Cu) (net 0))
 (segment (start 165.05 92.78) (end 169.27 97) (width 0.25) (layer F.Cu) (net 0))
 (segment (start 170.95 91.925) (end 170.95 96.14) (width 0.25) (layer F.Cu) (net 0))
 (segment (start 170.95 96.14) (end 171.81 97) (width 0.25) (layer F.Cu) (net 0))
 (segment (start 161 100.25) (end 161 98.89) (width 0.25) (layer F.Cu) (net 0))
 (segment (start 161 98.89) (end 159.11 97) (width 0.25) (layer F.Cu) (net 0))
 (segment (start 163 100.25) (end 163 98.35) (width 0.25) (layer F.Cu) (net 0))
 (segment (start 163 98.35) (end 161.65 97) (width 0.25) (layer F.Cu) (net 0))
 (segment (start 165 100.25) (end 165 97.81) (width 0.25) (layer F.Cu) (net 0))
 (segment (start 165 97.81) (end 164.19 97) (width 0.25) (layer F.Cu) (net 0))
 (segment (start 167 100.25) (end 167 97.27) (width 0.25) (layer F.Cu) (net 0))
 (segment (start 167 97.27) (end 166.73 97) (width 0.25) (layer F.Cu) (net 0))
 (segment (start 161 104.25) (end 161 101.75) (width 0.25) (layer F.Cu) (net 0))
 (segment (start 163 104.25) (end 163 101.75) (width 0.25) (layer F.Cu) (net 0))
 (segment (start 165 104.25) (end 165 101.75) (width 0.25) (layer F.Cu) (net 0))
 (segment (start 167 104.25) (end 167 101.75) (width 0.25) (layer F.Cu) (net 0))
 (segment (start 169 104.25) (end 169 101.75) (width 0.25) (layer F.Cu) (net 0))
 (segment (start 171 104.25) (end 171 101.75) (width 0.25) (layer F.Cu) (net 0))
 (segment (start 173 104.25) (end 173 101.75) (width 0.25) (layer F.Cu) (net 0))
 (segment (start 175 104.25) (end 175 101.75) (width 0.25) (layer F.Cu) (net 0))
 (segment (start 175 100.25) (end 175 98.89) (width 0.25) (layer F.Cu) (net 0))
 (segment (start 175 98.89) (end 176.89 97) (width 0.25) (layer F.Cu) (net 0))
 (segment (start 173 100.25) (end 173 98.35) (width 0.25) (layer F.Cu) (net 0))
 (segment (start 173 98.35) (end 174.35 97) (width 0.25) (layer F.Cu) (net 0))
 (segment (start 171 100.25) (end 171 97.81) (width 0.25) (layer F.Cu) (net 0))
 (segment (start 171 97.81) (end 171.81 97) (width 0.25) (layer F.Cu) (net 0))
 (segment (start 169 100.25) (end 169 97.27) (width 0.25) (layer F.Cu) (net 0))
 (segment (start 169 97.27) (end 169.27 97) (width 0.25) (layer F.Cu) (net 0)))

